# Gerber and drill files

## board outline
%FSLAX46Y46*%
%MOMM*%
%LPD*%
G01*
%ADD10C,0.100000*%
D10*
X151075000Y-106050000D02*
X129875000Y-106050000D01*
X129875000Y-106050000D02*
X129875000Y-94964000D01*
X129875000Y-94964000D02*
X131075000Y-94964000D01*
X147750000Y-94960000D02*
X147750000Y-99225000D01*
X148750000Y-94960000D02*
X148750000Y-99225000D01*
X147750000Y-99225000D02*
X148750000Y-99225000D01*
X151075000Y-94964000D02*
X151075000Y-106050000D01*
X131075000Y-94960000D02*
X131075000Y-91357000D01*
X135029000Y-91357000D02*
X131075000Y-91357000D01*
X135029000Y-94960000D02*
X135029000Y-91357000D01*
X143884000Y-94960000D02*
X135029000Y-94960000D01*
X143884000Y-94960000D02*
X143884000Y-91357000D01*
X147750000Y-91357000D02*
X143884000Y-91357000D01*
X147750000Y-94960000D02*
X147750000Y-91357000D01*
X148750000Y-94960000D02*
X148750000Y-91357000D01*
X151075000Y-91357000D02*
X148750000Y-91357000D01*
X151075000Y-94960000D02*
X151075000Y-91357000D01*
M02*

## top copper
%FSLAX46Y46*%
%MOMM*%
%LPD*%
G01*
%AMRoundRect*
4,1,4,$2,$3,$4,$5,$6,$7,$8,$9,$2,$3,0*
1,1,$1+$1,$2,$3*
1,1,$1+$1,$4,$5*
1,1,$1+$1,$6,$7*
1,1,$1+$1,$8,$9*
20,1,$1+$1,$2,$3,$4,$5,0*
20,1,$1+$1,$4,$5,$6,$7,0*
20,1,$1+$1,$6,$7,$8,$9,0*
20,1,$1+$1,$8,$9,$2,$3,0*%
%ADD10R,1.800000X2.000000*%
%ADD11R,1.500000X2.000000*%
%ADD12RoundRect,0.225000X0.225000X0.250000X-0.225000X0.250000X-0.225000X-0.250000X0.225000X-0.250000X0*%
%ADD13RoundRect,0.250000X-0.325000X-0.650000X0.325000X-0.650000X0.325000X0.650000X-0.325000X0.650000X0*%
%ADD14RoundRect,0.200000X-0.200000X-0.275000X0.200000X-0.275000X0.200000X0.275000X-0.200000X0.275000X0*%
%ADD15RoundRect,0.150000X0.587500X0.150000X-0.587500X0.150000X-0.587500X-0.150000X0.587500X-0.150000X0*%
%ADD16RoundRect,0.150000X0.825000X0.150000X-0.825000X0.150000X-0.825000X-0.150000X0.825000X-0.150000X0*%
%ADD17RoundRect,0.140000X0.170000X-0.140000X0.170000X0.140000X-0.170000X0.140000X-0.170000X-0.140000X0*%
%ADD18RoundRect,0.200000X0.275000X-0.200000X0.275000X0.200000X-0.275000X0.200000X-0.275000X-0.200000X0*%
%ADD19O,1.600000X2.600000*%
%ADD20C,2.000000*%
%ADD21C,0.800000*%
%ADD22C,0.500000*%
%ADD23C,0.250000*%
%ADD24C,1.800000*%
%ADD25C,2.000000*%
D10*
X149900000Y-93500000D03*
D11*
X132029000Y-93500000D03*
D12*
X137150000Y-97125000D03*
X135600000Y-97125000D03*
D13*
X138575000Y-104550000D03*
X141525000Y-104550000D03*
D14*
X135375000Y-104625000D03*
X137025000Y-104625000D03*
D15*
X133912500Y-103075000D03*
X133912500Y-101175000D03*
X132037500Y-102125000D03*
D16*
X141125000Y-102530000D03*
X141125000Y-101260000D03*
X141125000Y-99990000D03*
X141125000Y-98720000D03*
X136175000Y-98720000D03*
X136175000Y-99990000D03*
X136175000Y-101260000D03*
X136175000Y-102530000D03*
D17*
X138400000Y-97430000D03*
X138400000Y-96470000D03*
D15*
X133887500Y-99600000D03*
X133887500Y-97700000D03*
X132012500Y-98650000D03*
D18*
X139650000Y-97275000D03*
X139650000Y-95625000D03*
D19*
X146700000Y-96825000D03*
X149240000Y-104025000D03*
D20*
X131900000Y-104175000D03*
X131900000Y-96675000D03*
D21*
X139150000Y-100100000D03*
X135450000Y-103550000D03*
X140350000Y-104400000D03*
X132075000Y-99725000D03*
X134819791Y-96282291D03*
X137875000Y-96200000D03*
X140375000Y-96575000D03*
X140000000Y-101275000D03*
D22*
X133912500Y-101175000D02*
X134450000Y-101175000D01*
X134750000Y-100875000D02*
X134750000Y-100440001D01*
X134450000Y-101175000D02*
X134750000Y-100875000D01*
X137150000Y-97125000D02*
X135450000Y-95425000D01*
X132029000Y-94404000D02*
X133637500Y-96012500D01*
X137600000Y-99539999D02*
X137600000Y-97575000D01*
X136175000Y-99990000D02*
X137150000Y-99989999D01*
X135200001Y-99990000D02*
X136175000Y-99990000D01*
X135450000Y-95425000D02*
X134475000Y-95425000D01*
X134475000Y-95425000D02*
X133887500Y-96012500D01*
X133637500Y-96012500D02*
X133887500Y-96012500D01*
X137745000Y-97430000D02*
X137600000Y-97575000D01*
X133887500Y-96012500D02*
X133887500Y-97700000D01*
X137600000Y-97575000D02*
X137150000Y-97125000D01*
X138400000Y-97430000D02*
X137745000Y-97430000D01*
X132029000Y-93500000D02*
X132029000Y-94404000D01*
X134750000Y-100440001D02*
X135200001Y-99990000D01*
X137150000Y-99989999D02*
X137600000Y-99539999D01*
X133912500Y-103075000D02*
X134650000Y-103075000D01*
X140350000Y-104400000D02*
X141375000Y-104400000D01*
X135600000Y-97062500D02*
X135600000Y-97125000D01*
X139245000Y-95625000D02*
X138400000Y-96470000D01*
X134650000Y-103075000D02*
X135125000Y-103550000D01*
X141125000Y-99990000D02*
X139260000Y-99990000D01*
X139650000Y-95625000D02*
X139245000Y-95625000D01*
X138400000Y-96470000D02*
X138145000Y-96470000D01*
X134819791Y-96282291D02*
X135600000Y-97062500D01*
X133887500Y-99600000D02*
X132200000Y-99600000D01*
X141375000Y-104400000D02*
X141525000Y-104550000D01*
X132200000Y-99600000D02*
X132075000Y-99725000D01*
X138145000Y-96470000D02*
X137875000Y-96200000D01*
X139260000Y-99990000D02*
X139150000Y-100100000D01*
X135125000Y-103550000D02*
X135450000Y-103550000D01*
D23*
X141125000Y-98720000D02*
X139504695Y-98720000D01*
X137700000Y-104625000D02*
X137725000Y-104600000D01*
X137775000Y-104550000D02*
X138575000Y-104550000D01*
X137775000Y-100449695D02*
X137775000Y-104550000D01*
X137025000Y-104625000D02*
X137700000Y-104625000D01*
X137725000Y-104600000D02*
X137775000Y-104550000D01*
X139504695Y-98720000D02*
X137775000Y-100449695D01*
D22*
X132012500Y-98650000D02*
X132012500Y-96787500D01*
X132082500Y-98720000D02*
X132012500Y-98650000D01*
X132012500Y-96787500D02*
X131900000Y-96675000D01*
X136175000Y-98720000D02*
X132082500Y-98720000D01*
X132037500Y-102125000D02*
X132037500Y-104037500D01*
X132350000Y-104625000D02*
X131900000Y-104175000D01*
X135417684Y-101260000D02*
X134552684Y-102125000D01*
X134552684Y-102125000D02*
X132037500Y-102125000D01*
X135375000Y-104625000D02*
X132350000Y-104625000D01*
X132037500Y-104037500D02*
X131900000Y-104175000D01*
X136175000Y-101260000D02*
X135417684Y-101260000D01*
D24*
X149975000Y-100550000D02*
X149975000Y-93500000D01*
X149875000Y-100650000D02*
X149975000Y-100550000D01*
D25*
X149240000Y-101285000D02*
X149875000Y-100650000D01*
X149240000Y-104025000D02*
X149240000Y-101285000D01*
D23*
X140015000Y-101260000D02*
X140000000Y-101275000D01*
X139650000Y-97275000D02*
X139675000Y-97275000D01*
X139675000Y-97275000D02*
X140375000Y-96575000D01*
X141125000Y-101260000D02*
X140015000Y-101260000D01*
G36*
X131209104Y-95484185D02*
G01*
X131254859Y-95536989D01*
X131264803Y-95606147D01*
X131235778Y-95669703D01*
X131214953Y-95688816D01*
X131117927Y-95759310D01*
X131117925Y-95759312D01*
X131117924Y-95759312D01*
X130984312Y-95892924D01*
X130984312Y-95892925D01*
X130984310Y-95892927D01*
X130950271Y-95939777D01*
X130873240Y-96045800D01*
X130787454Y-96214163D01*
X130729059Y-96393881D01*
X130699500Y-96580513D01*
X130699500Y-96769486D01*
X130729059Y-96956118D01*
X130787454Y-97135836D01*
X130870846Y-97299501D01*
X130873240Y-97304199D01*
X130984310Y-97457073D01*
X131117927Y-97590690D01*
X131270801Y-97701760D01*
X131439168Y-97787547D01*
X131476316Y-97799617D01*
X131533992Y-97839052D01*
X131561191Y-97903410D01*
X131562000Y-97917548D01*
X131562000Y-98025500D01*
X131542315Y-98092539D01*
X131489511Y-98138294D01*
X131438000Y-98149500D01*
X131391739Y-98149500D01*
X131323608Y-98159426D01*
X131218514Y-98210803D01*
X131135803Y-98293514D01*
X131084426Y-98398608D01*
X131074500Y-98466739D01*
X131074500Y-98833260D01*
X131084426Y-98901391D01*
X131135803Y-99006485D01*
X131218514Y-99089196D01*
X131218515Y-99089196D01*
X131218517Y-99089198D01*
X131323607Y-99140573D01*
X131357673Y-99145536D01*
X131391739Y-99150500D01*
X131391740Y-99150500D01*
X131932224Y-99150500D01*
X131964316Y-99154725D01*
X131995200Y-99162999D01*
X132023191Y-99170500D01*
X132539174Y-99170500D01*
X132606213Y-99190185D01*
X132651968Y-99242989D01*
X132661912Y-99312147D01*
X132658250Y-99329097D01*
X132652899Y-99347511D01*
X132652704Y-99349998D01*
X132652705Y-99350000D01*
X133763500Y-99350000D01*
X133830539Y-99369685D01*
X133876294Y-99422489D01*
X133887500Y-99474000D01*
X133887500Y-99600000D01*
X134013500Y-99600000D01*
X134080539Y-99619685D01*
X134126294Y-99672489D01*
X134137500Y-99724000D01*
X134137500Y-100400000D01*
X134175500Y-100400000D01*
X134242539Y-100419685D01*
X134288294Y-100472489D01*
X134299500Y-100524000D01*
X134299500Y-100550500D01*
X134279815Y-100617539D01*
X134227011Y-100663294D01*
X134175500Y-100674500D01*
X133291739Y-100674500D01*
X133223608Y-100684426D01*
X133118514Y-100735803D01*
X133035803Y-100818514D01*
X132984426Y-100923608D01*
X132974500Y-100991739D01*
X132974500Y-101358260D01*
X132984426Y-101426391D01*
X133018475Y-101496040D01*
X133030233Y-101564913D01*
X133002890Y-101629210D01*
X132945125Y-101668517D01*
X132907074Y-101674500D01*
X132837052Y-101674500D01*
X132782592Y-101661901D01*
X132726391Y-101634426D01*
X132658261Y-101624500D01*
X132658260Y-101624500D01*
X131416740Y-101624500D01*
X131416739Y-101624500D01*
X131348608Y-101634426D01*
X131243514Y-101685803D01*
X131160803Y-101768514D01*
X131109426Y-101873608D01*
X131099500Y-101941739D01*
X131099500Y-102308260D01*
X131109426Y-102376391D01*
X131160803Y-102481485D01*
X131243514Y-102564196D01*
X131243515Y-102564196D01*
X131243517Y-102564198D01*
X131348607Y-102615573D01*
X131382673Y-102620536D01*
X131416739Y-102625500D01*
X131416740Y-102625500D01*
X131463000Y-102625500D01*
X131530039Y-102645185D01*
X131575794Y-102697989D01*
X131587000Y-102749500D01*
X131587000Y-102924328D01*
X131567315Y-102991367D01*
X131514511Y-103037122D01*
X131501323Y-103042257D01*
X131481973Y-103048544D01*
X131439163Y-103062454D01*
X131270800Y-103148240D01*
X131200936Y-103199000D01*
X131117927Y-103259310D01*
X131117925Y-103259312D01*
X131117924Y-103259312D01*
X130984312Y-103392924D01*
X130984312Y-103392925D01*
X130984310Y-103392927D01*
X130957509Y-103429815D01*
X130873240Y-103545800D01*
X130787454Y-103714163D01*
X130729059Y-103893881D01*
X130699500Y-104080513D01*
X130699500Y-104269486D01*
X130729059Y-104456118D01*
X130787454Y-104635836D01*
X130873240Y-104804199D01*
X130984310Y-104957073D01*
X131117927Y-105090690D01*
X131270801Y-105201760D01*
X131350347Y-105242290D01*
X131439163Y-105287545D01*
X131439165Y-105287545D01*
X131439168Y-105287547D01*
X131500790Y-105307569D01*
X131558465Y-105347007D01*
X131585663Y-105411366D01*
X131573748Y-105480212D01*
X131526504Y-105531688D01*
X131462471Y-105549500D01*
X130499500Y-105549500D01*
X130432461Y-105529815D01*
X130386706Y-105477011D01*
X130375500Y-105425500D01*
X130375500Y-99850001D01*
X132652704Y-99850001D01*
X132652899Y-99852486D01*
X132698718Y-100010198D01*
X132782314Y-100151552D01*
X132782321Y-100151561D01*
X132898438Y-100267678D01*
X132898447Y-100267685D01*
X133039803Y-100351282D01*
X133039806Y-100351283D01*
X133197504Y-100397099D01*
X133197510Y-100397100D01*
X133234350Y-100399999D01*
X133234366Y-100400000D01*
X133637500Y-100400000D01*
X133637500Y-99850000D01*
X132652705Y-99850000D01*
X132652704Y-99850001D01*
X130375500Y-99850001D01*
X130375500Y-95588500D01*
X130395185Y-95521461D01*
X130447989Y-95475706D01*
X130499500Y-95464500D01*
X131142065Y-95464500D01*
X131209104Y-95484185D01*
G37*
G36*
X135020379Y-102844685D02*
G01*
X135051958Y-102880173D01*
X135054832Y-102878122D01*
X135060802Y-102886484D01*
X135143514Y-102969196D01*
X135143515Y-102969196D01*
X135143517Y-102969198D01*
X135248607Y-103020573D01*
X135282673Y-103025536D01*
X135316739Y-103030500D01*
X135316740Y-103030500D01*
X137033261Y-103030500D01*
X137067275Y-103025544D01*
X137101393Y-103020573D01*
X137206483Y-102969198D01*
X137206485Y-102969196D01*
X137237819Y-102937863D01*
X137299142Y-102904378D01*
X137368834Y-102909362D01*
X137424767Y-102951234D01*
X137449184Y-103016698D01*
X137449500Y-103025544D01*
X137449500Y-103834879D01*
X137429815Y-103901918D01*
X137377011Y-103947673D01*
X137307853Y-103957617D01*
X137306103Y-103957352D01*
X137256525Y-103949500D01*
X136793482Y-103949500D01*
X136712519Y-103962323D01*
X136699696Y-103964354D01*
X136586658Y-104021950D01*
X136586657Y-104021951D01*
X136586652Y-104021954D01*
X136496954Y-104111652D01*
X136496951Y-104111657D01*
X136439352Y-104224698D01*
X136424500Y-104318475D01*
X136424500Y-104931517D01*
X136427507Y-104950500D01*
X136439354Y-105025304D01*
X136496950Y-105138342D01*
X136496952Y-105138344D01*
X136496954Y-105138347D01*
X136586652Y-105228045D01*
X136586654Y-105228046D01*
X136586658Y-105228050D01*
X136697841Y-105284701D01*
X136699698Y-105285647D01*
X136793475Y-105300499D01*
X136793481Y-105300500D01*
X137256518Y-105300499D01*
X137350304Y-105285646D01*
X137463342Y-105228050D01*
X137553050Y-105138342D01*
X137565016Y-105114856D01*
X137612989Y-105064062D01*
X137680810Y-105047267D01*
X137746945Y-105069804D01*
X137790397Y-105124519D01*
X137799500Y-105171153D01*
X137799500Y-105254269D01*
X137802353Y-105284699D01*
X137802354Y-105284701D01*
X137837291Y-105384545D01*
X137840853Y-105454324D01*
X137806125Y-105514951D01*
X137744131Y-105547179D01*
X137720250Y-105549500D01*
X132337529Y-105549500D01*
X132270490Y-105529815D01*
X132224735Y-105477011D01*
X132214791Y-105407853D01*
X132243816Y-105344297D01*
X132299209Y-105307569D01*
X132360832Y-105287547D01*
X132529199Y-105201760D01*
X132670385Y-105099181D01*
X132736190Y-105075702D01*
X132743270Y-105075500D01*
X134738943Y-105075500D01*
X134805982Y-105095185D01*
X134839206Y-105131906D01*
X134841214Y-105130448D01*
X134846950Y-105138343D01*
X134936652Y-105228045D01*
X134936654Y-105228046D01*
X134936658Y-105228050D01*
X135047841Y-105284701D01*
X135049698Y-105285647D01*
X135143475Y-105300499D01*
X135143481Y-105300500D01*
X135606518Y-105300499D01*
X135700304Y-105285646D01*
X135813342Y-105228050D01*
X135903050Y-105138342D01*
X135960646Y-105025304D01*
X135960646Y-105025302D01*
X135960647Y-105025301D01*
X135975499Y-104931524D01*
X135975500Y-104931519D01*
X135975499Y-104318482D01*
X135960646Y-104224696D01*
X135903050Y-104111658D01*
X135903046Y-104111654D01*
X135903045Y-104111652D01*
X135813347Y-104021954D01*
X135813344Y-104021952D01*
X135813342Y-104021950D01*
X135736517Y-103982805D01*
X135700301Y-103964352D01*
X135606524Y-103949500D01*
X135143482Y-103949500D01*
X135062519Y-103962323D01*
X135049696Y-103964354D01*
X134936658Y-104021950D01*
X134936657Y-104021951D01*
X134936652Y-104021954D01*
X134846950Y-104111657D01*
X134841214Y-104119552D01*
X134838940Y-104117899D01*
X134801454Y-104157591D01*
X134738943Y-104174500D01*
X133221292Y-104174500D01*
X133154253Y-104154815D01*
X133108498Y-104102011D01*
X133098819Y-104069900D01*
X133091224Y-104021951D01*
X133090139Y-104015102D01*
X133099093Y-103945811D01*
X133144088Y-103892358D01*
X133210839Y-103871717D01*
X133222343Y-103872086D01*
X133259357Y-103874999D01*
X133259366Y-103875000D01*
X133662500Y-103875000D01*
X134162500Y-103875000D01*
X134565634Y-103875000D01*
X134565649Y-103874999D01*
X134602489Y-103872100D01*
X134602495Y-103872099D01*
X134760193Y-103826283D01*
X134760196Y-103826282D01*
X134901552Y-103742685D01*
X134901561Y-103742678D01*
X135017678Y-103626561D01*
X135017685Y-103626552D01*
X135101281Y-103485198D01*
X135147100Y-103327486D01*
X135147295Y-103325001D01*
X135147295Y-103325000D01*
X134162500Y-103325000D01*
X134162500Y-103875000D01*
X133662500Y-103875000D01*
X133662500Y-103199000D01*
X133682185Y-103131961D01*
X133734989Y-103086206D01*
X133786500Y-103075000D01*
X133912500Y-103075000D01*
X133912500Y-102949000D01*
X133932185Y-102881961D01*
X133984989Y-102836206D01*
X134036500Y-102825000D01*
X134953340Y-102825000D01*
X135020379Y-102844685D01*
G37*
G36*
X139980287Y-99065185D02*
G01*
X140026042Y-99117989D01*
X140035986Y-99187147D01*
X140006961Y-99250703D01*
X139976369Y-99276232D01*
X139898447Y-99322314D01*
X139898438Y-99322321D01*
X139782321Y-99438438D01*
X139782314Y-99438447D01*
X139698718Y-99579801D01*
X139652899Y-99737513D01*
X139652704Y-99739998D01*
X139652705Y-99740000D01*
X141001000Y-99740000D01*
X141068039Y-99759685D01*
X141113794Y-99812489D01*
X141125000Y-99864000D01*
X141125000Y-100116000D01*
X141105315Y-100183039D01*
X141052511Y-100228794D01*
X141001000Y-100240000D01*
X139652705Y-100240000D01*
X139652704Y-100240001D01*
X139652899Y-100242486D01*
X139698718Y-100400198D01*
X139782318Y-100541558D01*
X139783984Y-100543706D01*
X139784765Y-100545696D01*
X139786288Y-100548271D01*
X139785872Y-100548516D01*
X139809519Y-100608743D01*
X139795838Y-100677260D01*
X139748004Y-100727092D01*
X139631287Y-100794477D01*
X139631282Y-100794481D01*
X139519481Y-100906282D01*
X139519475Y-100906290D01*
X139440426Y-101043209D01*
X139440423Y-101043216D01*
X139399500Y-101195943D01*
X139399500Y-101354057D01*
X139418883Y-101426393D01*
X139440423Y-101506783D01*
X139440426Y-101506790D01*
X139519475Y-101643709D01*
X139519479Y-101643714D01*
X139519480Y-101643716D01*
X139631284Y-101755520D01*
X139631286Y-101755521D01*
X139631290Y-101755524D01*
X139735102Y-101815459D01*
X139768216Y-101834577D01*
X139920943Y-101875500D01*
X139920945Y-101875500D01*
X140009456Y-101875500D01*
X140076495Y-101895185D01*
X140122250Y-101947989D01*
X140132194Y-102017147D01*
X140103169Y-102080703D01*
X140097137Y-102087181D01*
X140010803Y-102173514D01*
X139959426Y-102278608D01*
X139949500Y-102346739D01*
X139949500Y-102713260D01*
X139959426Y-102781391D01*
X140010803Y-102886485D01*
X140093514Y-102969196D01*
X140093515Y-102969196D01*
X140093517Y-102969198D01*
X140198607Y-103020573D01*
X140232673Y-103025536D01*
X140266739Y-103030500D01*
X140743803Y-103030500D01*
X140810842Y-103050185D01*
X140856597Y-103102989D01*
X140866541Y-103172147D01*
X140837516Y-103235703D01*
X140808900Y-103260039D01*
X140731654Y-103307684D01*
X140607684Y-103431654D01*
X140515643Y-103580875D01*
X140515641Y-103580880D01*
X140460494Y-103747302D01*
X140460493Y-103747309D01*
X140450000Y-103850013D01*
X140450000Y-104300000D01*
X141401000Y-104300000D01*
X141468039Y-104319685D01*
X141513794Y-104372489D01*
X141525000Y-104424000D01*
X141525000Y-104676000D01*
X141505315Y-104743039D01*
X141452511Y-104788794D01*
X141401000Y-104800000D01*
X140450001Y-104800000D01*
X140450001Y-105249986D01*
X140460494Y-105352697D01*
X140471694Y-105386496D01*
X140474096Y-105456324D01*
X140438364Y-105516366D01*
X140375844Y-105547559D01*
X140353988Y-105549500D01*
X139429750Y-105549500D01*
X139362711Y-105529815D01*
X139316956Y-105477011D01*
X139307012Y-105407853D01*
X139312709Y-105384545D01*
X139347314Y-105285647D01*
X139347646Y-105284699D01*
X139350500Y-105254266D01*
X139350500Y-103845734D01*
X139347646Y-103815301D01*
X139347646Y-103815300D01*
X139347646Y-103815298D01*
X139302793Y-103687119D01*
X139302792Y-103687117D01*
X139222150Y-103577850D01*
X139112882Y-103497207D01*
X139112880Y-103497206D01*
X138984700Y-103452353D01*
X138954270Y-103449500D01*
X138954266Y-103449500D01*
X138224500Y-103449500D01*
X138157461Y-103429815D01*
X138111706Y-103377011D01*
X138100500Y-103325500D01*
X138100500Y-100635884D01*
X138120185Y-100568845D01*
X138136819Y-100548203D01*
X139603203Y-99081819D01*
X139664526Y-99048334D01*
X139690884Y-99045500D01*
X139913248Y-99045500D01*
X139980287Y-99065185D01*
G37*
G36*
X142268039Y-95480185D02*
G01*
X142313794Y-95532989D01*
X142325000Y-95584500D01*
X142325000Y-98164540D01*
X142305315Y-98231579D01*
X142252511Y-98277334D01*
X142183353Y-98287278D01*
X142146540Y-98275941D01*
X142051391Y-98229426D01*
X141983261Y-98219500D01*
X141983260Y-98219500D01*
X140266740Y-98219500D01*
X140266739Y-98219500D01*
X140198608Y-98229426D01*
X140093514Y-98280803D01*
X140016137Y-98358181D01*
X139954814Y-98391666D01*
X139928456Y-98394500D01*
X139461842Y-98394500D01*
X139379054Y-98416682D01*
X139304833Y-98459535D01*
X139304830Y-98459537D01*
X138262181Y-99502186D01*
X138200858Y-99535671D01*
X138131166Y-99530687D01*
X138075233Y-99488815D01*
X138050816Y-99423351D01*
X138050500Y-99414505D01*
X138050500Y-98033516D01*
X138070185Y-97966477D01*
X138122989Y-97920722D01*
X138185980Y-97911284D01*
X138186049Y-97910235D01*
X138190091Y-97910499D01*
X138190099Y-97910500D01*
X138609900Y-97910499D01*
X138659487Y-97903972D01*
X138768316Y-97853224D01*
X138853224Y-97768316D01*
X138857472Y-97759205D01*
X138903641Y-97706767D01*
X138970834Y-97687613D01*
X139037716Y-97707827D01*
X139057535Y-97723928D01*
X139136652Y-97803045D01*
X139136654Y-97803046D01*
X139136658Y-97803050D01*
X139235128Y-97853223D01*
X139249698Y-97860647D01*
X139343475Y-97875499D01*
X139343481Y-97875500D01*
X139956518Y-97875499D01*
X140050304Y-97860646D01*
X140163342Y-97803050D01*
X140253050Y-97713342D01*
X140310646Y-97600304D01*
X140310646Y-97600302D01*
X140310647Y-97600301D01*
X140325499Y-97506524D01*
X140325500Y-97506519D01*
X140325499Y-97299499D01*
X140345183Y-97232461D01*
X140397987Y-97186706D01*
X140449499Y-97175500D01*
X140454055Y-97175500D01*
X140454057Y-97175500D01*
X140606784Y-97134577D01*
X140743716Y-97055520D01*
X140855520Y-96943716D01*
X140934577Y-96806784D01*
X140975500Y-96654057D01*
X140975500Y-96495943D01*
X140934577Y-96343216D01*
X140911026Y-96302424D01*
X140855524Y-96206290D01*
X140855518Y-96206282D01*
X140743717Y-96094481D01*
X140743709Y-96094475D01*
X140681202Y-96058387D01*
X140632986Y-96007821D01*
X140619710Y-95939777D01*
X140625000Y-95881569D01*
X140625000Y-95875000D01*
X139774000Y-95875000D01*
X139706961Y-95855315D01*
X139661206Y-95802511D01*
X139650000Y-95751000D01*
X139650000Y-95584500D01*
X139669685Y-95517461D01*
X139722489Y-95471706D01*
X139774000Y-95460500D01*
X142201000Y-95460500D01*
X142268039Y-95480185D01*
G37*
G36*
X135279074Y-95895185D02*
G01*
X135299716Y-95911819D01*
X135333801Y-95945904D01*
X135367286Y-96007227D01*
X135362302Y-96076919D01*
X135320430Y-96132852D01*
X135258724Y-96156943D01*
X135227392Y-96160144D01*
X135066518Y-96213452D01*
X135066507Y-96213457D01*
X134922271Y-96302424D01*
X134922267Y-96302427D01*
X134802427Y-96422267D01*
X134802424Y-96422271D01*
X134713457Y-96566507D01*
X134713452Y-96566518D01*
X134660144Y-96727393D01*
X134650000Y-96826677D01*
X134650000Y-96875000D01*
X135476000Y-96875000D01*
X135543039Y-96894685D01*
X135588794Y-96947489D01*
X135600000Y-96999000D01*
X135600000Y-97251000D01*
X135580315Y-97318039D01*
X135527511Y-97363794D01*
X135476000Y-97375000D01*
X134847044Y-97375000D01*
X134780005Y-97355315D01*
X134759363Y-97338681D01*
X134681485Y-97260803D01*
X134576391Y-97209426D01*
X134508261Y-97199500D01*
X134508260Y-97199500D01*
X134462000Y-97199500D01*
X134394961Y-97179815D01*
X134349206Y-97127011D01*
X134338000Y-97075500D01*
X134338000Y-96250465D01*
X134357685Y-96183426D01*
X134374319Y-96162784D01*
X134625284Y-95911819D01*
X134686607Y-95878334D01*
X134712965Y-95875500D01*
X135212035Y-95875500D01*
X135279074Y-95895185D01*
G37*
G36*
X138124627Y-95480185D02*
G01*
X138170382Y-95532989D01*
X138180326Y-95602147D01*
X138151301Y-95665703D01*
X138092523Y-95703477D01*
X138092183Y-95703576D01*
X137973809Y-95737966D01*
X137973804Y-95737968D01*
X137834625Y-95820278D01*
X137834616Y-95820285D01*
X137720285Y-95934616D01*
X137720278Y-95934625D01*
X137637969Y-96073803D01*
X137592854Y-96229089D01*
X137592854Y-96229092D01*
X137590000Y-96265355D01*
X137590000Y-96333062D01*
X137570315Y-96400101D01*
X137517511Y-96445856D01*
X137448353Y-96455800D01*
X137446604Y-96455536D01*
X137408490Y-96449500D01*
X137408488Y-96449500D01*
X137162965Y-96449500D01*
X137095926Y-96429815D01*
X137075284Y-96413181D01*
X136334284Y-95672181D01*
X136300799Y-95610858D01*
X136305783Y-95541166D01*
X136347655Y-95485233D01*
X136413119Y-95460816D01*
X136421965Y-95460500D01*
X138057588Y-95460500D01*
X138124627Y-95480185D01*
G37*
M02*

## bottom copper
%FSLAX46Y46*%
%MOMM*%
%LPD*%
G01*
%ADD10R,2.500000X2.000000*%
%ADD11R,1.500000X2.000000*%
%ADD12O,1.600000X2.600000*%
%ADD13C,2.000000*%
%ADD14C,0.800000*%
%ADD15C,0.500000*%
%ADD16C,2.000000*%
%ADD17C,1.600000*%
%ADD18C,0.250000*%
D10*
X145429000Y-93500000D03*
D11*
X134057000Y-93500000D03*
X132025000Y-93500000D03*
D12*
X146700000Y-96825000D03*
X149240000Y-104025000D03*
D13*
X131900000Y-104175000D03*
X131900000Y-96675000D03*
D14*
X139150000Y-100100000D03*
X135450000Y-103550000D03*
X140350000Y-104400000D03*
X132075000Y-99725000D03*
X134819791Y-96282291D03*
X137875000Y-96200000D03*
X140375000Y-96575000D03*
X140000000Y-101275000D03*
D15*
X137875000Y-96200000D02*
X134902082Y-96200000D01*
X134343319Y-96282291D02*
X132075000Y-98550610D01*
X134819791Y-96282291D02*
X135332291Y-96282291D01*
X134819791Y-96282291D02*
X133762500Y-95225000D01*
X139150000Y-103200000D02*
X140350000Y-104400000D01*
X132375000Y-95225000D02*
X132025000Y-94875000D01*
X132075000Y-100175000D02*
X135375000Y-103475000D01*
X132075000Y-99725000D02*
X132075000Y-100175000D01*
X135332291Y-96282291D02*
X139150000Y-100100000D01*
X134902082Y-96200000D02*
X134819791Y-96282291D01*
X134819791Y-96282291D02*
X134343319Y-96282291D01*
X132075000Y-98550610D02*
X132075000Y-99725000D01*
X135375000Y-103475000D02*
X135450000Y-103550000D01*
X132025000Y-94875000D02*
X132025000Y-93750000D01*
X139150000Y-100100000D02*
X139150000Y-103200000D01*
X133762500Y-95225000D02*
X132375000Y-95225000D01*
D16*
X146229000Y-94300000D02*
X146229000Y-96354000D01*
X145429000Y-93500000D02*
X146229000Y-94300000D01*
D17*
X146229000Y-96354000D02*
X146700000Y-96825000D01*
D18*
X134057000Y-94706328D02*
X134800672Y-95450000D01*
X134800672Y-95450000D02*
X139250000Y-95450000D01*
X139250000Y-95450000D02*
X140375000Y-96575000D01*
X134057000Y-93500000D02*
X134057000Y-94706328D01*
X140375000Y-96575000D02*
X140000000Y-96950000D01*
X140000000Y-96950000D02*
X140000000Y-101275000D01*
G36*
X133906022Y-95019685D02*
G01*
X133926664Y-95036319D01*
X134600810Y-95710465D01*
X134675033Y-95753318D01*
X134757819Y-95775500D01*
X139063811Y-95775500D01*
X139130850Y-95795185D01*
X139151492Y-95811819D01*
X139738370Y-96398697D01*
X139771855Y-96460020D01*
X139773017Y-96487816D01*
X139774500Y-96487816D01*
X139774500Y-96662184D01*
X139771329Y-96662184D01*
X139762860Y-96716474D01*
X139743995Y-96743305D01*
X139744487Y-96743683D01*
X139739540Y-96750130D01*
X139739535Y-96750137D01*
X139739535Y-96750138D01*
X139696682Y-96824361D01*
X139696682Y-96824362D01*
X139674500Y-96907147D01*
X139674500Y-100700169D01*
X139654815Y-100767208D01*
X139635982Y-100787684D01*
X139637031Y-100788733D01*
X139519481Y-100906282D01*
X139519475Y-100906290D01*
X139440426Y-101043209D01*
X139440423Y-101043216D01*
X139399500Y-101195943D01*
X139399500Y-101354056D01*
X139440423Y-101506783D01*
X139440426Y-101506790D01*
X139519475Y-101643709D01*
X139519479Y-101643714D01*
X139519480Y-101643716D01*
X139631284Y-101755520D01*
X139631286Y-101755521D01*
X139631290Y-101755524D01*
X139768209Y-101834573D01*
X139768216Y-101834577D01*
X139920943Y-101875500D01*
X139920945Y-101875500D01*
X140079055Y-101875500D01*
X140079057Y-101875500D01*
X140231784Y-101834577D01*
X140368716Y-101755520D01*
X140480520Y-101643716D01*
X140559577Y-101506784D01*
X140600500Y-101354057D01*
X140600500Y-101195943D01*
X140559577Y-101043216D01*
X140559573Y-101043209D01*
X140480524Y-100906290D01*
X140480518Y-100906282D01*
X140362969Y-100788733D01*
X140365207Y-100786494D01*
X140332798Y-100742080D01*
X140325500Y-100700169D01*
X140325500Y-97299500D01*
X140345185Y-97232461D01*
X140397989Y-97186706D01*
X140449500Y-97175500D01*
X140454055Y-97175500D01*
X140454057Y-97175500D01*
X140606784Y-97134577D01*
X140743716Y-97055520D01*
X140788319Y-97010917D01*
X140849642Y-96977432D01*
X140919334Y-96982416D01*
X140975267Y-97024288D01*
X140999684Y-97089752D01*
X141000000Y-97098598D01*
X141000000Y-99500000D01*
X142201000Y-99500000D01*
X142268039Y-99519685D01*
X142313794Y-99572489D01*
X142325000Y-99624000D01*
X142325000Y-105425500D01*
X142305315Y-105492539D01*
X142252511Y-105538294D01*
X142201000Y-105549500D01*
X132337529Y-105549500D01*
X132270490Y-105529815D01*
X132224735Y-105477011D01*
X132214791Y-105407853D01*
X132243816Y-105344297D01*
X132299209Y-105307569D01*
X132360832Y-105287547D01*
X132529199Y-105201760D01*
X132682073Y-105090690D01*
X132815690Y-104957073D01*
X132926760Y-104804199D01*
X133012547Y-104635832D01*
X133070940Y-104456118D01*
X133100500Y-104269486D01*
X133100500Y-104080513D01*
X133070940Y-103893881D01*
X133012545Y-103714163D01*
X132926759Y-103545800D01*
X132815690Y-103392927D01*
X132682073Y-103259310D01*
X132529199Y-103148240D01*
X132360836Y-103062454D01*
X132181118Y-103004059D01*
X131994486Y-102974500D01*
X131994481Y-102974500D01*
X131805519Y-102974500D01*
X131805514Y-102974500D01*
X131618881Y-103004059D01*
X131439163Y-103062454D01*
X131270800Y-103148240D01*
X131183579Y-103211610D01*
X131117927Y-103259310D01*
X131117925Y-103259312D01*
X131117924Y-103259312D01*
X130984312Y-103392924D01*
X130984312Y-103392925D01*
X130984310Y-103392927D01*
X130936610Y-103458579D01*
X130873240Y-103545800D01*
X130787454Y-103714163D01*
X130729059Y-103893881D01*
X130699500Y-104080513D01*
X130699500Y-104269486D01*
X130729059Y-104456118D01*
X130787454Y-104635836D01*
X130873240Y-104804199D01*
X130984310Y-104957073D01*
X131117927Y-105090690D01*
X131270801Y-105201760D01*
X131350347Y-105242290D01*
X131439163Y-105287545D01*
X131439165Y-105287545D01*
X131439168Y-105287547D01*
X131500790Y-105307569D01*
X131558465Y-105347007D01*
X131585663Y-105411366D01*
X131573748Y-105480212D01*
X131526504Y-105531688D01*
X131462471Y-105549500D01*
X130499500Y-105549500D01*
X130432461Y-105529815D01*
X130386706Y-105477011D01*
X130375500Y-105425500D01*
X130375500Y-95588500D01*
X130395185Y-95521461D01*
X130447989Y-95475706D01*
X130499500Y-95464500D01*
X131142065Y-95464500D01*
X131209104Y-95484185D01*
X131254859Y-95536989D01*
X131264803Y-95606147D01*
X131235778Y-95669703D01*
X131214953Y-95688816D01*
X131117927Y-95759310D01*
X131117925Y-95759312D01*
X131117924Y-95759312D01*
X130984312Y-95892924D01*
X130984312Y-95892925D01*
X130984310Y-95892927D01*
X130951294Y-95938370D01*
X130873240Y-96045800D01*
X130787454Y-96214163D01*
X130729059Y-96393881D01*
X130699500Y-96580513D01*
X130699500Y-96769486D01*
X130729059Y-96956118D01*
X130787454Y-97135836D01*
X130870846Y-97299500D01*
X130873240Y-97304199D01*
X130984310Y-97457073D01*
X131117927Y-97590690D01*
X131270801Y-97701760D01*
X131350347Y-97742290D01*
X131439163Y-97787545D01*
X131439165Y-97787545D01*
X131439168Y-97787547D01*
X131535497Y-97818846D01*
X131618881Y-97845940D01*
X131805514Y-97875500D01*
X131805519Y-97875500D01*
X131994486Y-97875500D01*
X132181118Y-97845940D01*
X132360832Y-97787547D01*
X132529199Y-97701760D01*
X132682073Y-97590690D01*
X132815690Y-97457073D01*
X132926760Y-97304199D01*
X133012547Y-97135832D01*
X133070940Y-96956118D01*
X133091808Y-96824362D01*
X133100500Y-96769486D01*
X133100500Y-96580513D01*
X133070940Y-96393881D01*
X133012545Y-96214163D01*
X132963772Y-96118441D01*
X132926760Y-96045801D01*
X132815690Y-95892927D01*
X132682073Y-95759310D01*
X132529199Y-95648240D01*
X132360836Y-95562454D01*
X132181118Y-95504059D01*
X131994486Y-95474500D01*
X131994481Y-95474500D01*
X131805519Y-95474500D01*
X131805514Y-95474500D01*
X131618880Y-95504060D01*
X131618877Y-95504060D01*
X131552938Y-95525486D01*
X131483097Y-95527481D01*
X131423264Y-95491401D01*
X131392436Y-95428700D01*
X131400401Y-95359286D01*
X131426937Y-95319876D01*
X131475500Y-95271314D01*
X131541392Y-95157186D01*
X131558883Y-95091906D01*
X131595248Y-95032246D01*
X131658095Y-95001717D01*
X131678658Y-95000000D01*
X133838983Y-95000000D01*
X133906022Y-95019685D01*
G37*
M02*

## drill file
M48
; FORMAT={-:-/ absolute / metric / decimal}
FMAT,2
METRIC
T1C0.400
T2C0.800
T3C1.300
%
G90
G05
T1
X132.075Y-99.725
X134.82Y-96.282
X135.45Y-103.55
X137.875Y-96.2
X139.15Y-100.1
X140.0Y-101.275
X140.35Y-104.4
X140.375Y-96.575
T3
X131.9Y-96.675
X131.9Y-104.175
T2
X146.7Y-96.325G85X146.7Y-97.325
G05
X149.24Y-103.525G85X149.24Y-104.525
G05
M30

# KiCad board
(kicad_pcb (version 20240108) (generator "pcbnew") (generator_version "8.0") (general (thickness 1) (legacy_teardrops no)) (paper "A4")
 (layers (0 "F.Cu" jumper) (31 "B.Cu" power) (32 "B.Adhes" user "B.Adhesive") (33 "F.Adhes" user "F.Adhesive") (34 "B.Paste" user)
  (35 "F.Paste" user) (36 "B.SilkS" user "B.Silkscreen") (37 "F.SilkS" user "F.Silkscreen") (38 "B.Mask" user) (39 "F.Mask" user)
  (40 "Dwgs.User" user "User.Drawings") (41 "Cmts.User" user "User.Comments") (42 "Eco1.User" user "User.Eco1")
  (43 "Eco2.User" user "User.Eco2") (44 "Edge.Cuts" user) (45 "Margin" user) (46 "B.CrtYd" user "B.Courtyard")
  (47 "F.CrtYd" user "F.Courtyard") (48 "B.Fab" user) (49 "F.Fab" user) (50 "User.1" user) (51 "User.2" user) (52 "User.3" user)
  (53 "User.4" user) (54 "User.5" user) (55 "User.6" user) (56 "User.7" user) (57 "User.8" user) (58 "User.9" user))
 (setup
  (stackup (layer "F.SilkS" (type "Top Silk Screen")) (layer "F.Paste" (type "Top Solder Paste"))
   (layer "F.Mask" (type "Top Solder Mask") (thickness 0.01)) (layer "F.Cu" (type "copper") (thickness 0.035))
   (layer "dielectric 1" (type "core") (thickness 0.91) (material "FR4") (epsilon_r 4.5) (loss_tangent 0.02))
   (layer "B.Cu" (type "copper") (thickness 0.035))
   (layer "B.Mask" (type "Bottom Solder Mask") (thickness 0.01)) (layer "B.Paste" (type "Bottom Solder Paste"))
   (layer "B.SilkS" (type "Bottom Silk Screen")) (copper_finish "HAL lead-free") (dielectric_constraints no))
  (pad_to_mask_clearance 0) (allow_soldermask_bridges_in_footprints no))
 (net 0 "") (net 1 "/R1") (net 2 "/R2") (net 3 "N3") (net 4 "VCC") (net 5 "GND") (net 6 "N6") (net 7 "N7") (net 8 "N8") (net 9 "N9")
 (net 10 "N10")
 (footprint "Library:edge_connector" (layer "F.Cu") (at 151.329 92.23 180)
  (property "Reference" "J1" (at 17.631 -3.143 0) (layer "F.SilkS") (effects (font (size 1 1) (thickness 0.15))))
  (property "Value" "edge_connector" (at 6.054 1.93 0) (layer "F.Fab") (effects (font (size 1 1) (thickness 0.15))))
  (fp_line (start 20.254 -2.73) (end 20.254 0.873) (stroke (width 0.1) (type solid)) (layer "Edge.Cuts"))
  (fp_line (start 16.3 0.873) (end 20.254 0.873) (stroke (width 0.1) (type solid)) (layer "Edge.Cuts"))
  (fp_line (start 16.3 -2.73) (end 16.3 0.873) (stroke (width 0.1) (type solid)) (layer "Edge.Cuts"))
  (fp_line (start 7.445 -2.73) (end 16.3 -2.73) (stroke (width 0.1) (type solid)) (layer "Edge.Cuts"))
  (fp_line (start 7.445 -2.73) (end 7.445 0.873) (stroke (width 0.1) (type solid)) (layer "Edge.Cuts"))
  (fp_line (start 3.579 0.873) (end 7.445 0.873) (stroke (width 0.1) (type solid)) (layer "Edge.Cuts"))
  (fp_line (start 3.579 -2.73) (end 3.579 0.873) (stroke (width 0.1) (type solid)) (layer "Edge.Cuts"))
  (fp_line (start 2.579 -2.73) (end 2.579 0.873) (stroke (width 0.1) (type solid)) (layer "Edge.Cuts"))
  (fp_line (start 0.254 0.873) (end 2.579 0.873) (stroke (width 0.1) (type solid)) (layer "Edge.Cuts"))
  (fp_line (start 0.254 -2.73) (end 0.254 0.873) (stroke (width 0.1) (type solid)) (layer "Edge.Cuts"))
  (pad "1" connect rect (at 1.429 -1.27 180) (size 1.8 2) (layers "F.Cu" "F.Mask") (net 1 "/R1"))
  (pad "2" connect rect (at 5.9 -1.27 180) (size 2.5 2) (layers "B.Cu" "B.Mask") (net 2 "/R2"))
  (pad "3" connect rect (at 17.272 -1.27 180) (size 1.5 2) (layers "B.Cu" "B.Mask") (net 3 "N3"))
  (pad "4" connect rect (at 19.3 -1.27 180) (size 1.5 2) (layers "F.Cu" "F.Mask") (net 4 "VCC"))
  (pad "5" connect rect (at 19.304 -1.27 180) (size 1.5 2) (layers "B.Cu" "B.Mask") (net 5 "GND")))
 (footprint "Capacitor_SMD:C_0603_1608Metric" (layer "F.Cu") (at 136.375 97.125 180)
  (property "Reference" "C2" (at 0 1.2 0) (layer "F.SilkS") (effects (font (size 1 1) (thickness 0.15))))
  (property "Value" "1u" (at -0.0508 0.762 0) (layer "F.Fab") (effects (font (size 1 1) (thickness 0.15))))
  (pad "1" smd roundrect (at -0.775 0 180) (size 0.9 0.95) (layers "F.Cu" "F.Paste" "F.Mask") (roundrect_rratio 0.25) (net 4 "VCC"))
  (pad "2" smd roundrect (at 0.775 0 180) (size 0.9 0.95) (layers "F.Cu" "F.Paste" "F.Mask") (roundrect_rratio 0.25) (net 5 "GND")))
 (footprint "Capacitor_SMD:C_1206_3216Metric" (layer "F.Cu") (at 140.05 104.55)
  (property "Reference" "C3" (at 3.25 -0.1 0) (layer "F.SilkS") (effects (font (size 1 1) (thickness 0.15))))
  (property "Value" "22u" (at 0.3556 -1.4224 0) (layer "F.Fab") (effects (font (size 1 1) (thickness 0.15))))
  (pad "1" smd roundrect (at -1.475 0) (size 1.15 1.8) (layers "F.Cu" "F.Paste" "F.Mask") (roundrect_rratio 0.2173913043) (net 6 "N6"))
  (pad "2" smd roundrect (at 1.475 0) (size 1.15 1.8) (layers "F.Cu" "F.Paste" "F.Mask") (roundrect_rratio 0.2173913043) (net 5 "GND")))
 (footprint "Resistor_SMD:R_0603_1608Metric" (layer "F.Cu") (at 136.2 104.625)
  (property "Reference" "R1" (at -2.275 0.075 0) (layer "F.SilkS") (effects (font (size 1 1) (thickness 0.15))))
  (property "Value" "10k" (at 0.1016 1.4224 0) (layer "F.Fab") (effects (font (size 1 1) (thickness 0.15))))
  (pad "1" smd roundrect (at -0.825 0) (size 0.8 0.95) (layers "F.Cu" "F.Paste" "F.Mask") (roundrect_rratio 0.25) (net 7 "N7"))
  (pad "2" smd roundrect (at 0.825 0) (size 0.8 0.95) (layers "F.Cu" "F.Paste" "F.Mask") (roundrect_rratio 0.25) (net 6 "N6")))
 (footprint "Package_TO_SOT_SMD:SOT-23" (layer "F.Cu") (at 132.975 102.125 180)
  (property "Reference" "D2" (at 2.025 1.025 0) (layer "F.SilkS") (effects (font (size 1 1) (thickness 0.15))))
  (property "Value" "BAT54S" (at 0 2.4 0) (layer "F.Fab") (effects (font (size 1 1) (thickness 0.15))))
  (pad "1" smd roundrect (at -0.9375 -0.95 180) (size 1.475 0.6) (layers "F.Cu" "F.Paste" "F.Mask") (roundrect_rratio 0.25) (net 5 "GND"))
  (pad "2" smd roundrect (at -0.9375 0.95 180) (size 1.475 0.6) (layers "F.Cu" "F.Paste" "F.Mask") (roundrect_rratio 0.25) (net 4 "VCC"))
  (pad "3" smd roundrect (at 0.9375 0 180) (size 1.475 0.6) (layers "F.Cu" "F.Paste" "F.Mask") (roundrect_rratio 0.25) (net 7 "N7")))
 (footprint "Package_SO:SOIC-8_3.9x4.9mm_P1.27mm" (layer "F.Cu") (at 138.65 100.625 180)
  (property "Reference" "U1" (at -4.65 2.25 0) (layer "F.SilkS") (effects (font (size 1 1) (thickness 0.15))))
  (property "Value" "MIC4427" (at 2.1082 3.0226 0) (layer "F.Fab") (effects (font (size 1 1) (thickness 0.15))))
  (pad "1" smd roundrect (at -2.475 -1.905 180) (size 1.95 0.6) (layers "F.Cu" "F.Paste" "F.Mask") (roundrect_rratio 0.25) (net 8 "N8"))
  (pad "2" smd roundrect (at -2.475 -0.635 180) (size 1.95 0.6) (layers "F.Cu" "F.Paste" "F.Mask") (roundrect_rratio 0.25) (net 3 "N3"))
  (pad "3" smd roundrect (at -2.475 0.635 180) (size 1.95 0.6) (layers "F.Cu" "F.Paste" "F.Mask") (roundrect_rratio 0.25) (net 5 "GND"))
  (pad "4" smd roundrect (at -2.475 1.905 180) (size 1.95 0.6) (layers "F.Cu" "F.Paste" "F.Mask") (roundrect_rratio 0.25) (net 6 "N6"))
  (pad "5" smd roundrect (at 2.475 1.905 180) (size 1.95 0.6) (layers "F.Cu" "F.Paste" "F.Mask") (roundrect_rratio 0.25) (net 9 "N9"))
  (pad "6" smd roundrect (at 2.475 0.635 180) (size 1.95 0.6) (layers "F.Cu" "F.Paste" "F.Mask") (roundrect_rratio 0.25) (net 4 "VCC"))
  (pad "7" smd roundrect (at 2.475 -0.635 180) (size 1.95 0.6) (layers "F.Cu" "F.Paste" "F.Mask") (roundrect_rratio 0.25) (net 7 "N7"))
  (pad "8" smd roundrect (at 2.475 -1.905 180) (size 1.95 0.6) (layers "F.Cu" "F.Paste" "F.Mask") (roundrect_rratio 0.25) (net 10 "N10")))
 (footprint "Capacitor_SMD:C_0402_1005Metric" (layer "F.Cu") (at 138.4 96.95 90)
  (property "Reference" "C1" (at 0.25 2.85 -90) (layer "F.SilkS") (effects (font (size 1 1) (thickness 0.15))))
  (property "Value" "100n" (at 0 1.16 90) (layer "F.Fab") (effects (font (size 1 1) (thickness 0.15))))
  (pad "1" smd roundrect (at -0.48 0 90) (size 0.56 0.62) (layers "F.Cu" "F.Paste" "F.Mask") (roundrect_rratio 0.25) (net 4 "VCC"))
  (pad "2" smd roundrect (at 0.48 0 90) (size 0.56 0.62) (layers "F.Cu" "F.Paste" "F.Mask") (roundrect_rratio 0.25) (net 5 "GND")))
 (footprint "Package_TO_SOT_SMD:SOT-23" (layer "F.Cu") (at 132.95 98.65 180)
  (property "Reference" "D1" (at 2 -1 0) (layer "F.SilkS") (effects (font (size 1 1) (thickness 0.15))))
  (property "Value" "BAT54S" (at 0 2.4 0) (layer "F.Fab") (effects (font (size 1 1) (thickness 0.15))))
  (pad "1" smd roundrect (at -0.9375 -0.95 180) (size 1.475 0.6) (layers "F.Cu" "F.Paste" "F.Mask") (roundrect_rratio 0.25) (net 5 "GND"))
  (pad "2" smd roundrect (at -0.9375 0.95 180) (size 1.475 0.6) (layers "F.Cu" "F.Paste" "F.Mask") (roundrect_rratio 0.25) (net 4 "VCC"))
  (pad "3" smd roundrect (at 0.9375 0 180) (size 1.475 0.6) (layers "F.Cu" "F.Paste" "F.Mask") (roundrect_rratio 0.25) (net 9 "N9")))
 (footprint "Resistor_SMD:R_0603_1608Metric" (layer "F.Cu") (at 139.65 96.45 90)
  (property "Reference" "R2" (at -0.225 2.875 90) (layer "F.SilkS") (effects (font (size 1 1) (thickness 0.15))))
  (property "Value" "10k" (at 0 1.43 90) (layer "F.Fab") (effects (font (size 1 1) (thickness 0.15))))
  (pad "1" smd roundrect (at -0.825 0 90) (size 0.8 0.95) (layers "F.Cu" "F.Paste" "F.Mask") (roundrect_rratio 0.25) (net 3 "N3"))
  (pad "2" smd roundrect (at 0.825 0 90) (size 0.8 0.95) (layers "F.Cu" "F.Paste" "F.Mask") (roundrect_rratio 0.25) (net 5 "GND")))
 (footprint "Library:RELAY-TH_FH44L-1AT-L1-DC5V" (layer "B.Cu") (at 140.57 100.425)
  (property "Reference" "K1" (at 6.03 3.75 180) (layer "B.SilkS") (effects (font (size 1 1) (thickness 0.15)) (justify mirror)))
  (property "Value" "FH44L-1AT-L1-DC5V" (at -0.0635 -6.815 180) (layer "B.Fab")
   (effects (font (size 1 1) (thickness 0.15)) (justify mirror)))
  (pad "13" thru_hole oval (at 6.13 -3.6) (size 1.6 2.6) (drill oval 0.8 1.8) (layers "*.Cu" "*.Mask") (remove_unused_layers no)
   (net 2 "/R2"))
  (pad "14" thru_hole oval (at 8.67 3.6) (size 1.6 2.6) (drill oval 0.8 1.8) (layers "*.Cu" "*.Mask") (remove_unused_layers no)
   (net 1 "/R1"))
  (pad "A1" thru_hole circle (at -8.67 3.75) (size 2 2) (drill 1.3) (layers "*.Cu" "*.Mask") (remove_unused_layers no) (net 7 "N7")
   (thermal_bridge_angle 90))
  (pad "A2" thru_hole circle (at -8.67 -3.75) (size 2 2) (drill 1.3) (layers "*.Cu" "*.Mask") (remove_unused_layers no) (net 9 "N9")
   (thermal_bridge_angle 90)))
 (gr_line (start 151.075 106.05) (end 129.875 106.05) (stroke (width 0.1) (type solid)) (layer "Edge.Cuts"))
 (gr_line (start 129.875 106.05) (end 129.875 94.964) (stroke (width 0.1) (type solid)) (layer "Edge.Cuts"))
 (gr_line (start 129.875 94.964) (end 131.075 94.964) (stroke (width 0.1) (type solid)) (layer "Edge.Cuts"))
 (gr_line (start 147.75 94.96) (end 147.75 99.225) (stroke (width 0.1) (type default)) (layer "Edge.Cuts"))
 (gr_line (start 148.75 94.96) (end 148.75 99.225) (stroke (width 0.1) (type default)) (layer "Edge.Cuts"))
 (gr_line (start 147.75 99.225) (end 148.75 99.225) (stroke (width 0.1) (type default)) (layer "Edge.Cuts"))
 (gr_line (start 151.075 94.964) (end 151.075 106.05) (stroke (width 0.1) (type solid)) (layer "Edge.Cuts"))
 (segment (start 133.9125 101.175) (end 134.45 101.175) (width 0.5) (layer "F.Cu") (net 4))
 (segment (start 134.75 100.875) (end 134.75 100.440001) (width 0.5) (layer "F.Cu") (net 4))
 (segment (start 134.45 101.175) (end 134.75 100.875) (width 0.5) (layer "F.Cu") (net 4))
 (segment (start 137.15 97.125) (end 135.45 95.425) (width 0.5) (layer "F.Cu") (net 4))
 (segment (start 132.029 94.404) (end 133.6375 96.0125) (width 0.5) (layer "F.Cu") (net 4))
 (segment (start 137.6 99.539999) (end 137.6 97.575) (width 0.5) (layer "F.Cu") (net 4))
 (segment (start 136.175 99.99) (end 137.15 99.989999) (width 0.5) (layer "F.Cu") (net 4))
 (segment (start 135.200001 99.99) (end 136.175 99.99) (width 0.5) (layer "F.Cu") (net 4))
 (segment (start 135.45 95.425) (end 134.475 95.425) (width 0.5) (layer "F.Cu") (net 4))
 (segment (start 134.475 95.425) (end 133.8875 96.0125) (width 0.5) (layer "F.Cu") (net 4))
 (segment (start 133.6375 96.0125) (end 133.8875 96.0125) (width 0.5) (layer "F.Cu") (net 4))
 (segment (start 137.745 97.43) (end 137.6 97.575) (width 0.5) (layer "F.Cu") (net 4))
 (segment (start 133.8875 96.0125) (end 133.8875 97.7) (width 0.5) (layer "F.Cu") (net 4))
 (segment (start 137.6 97.575) (end 137.15 97.125) (width 0.5) (layer "F.Cu") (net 4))
 (segment (start 138.4 97.43) (end 137.745 97.43) (width 0.5) (layer "F.Cu") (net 4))
 (segment (start 132.029 93.5) (end 132.029 94.404) (width 0.5) (layer "F.Cu") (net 4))
 (segment (start 134.75 100.440001) (end 135.200001 99.99) (width 0.5) (layer "F.Cu") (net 4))
 (segment (start 137.15 99.989999) (end 137.6 99.539999) (width 0.5) (layer "F.Cu") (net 4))
 (segment (start 133.9125 103.075) (end 134.65 103.075) (width 0.5) (layer "F.Cu") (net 5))
 (segment (start 140.35 104.4) (end 141.375 104.4) (width 0.5) (layer "F.Cu") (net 5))
 (segment (start 135.6 97.0625) (end 135.6 97.125) (width 0.5) (layer "F.Cu") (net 5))
 (segment (start 139.245 95.625) (end 138.4 96.47) (width 0.5) (layer "F.Cu") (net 5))
 (segment (start 134.65 103.075) (end 135.125 103.55) (width 0.5) (layer "F.Cu") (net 5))
 (segment (start 141.125 99.99) (end 139.26 99.99) (width 0.5) (layer "F.Cu") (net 5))
 (segment (start 139.65 95.625) (end 139.245 95.625) (width 0.5) (layer "F.Cu") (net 5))
 (segment (start 138.4 96.47) (end 138.145 96.47) (width 0.5) (layer "F.Cu") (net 5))
 (segment (start 134.819791 96.282291) (end 135.6 97.0625) (width 0.5) (layer "F.Cu") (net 5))
 (segment (start 133.8875 99.6) (end 132.2 99.6) (width 0.5) (layer "F.Cu") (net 5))
 (segment (start 141.375 104.4) (end 141.525 104.55) (width 0.5) (layer "F.Cu") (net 5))
 (segment (start 132.2 99.6) (end 132.075 99.725) (width 0.5) (layer "F.Cu") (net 5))
 (segment (start 138.145 96.47) (end 137.875 96.2) (width 0.5) (layer "F.Cu") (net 5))
 (segment (start 139.26 99.99) (end 139.15 100.1) (width 0.5) (layer "F.Cu") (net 5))
 (segment (start 135.125 103.55) (end 135.45 103.55) (width 0.5) (layer "F.Cu") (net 5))
 (via (at 139.15 100.1) (size 0.8) (drill 0.4) (layers "F.Cu" "B.Cu") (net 5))
 (via (at 135.45 103.55) (size 0.8) (drill 0.4) (layers "F.Cu" "B.Cu") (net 5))
 (via (at 140.35 104.4) (size 0.8) (drill 0.4) (layers "F.Cu" "B.Cu") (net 5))
 (via (at 132.075 99.725) (size 0.8) (drill 0.4) (layers "F.Cu" "B.Cu") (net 5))
 (via (at 134.819791 96.282291) (size 0.8) (drill 0.4) (layers "F.Cu" "B.Cu") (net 5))
 (via (at 137.875 96.2) (size 0.8) (drill 0.4) (layers "F.Cu" "B.Cu") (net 5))
 (segment (start 137.875 96.2) (end 134.902082 96.2) (width 0.5) (layer "B.Cu") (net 5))
 (segment (start 134.343319 96.282291) (end 132.075 98.55061) (width 0.5) (layer "B.Cu") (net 5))
 (segment (start 134.819791 96.282291) (end 135.332291 96.282291) (width 0.5) (layer "B.Cu") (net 5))
 (segment (start 134.819791 96.282291) (end 133.7625 95.225) (width 0.5) (layer "B.Cu") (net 5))
 (segment (start 139.15 103.2) (end 140.35 104.4) (width 0.5) (layer "B.Cu") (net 5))
 (segment (start 132.375 95.225) (end 132.025 94.875) (width 0.5) (layer "B.Cu") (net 5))
 (segment (start 132.075 100.175) (end 135.375 103.475) (width 0.5) (layer "B.Cu") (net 5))
 (segment (start 132.075 99.725) (end 132.075 100.175) (width 0.5) (layer "B.Cu") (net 5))
 (segment (start 135.332291 96.282291) (end 139.15 100.1) (width 0.5) (layer "B.Cu") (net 5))
 (segment (start 134.902082 96.2) (end 134.819791 96.282291) (width 0.5) (layer "B.Cu") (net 5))
 (segment (start 134.819791 96.282291) (end 134.343319 96.282291) (width 0.5) (layer "B.Cu") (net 5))
 (segment (start 132.075 98.55061) (end 132.075 99.725) (width 0.5) (layer "B.Cu") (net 5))
 (segment (start 135.375 103.475) (end 135.45 103.55) (width 0.5) (layer "B.Cu") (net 5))
 (segment (start 132.025 94.875) (end 132.025 93.75) (width 0.5) (layer "B.Cu") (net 5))
 (segment (start 139.15 100.1) (end 139.15 103.2) (width 0.5) (layer "B.Cu") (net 5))
 (segment (start 133.7625 95.225) (end 132.375 95.225) (width 0.5) (layer "B.Cu") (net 5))
 (segment (start 141.125 98.72) (end 139.504695 98.72) (width 0.25) (layer "F.Cu") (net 6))
 (segment (start 137.7 104.625) (end 137.725 104.6) (width 0.25) (layer "F.Cu") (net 6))
 (segment (start 137.775 104.55) (end 138.575 104.55) (width 0.25) (layer "F.Cu") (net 6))
 (segment (start 137.775 100.449695) (end 137.775 104.55) (width 0.25) (layer "F.Cu") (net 6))
 (segment (start 137.025 104.625) (end 137.7 104.625) (width 0.25) (layer "F.Cu") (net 6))
 (segment (start 137.725 104.6) (end 137.775 104.55) (width 0.25) (layer "F.Cu") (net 6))
 (segment (start 139.504695 98.72) (end 137.775 100.449695) (width 0.25) (layer "F.Cu") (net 6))
 (segment (start 132.0125 98.65) (end 132.0125 96.7875) (width 0.5) (layer "F.Cu") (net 9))
 (segment (start 132.0825 98.72) (end 132.0125 98.65) (width 0.5) (layer "F.Cu") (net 9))
 (segment (start 132.0125 96.7875) (end 131.9 96.675) (width 0.5) (layer "F.Cu") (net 9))
 (segment (start 136.175 98.72) (end 132.0825 98.72) (width 0.5) (layer "F.Cu") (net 9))
 (segment (start 132.0375 102.125) (end 132.0375 104.0375) (width 0.5) (layer "F.Cu") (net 7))
 (segment (start 132.35 104.625) (end 131.9 104.175) (width 0.5) (layer "F.Cu") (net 7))
 (segment (start 135.417684 101.26) (end 134.552684 102.125) (width 0.5) (layer "F.Cu") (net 7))
 (segment (start 134.552684 102.125) (end 132.0375 102.125) (width 0.5) (layer "F.Cu") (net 7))
 (segment (start 135.375 104.625) (end 132.35 104.625) (width 0.5) (layer "F.Cu") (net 7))
 (segment (start 132.0375 104.0375) (end 131.9 104.175) (width 0.5) (layer "F.Cu") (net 7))
 (segment (start 136.175 101.26) (end 135.417684 101.26) (width 0.5) (layer "F.Cu") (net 7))
 (segment (start 146.229 94.3) (end 146.229 96.354) (width 2) (layer "B.Cu") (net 2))
 (segment (start 145.429 93.5) (end 146.229 94.3) (width 2) (layer "B.Cu") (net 2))
 (segment (start 146.229 96.354) (end 146.7 96.825) (width 1.6) (layer "B.Cu") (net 2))
 (segment (start 149.975 100.55) (end 149.975 93.5) (width 1.8) (layer "F.Cu") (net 1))
 (segment (start 149.875 100.65) (end 149.975 100.55) (width 1.8) (layer "F.Cu") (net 1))
 (segment (start 149.24 101.285) (end 149.875 100.65) (width 2) (layer "F.Cu") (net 1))
 (segment (start 149.24 104.025) (end 149.24 101.285) (width 2) (layer "F.Cu") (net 1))
 (segment (start 140.015 101.26) (end 140 101.275) (width 0.25) (layer "F.Cu") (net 3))
 (segment (start 139.65 97.275) (end 139.675 97.275) (width 0.25) (layer "F.Cu") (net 3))
 (segment (start 139.675 97.275) (end 140.375 96.575) (width 0.25) (layer "F.Cu") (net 3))
 (segment (start 141.125 101.26) (end 140.015 101.26) (width 0.25) (layer "F.Cu") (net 3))
 (via (at 140.375 96.575) (size 0.8) (drill 0.4) (layers "F.Cu" "B.Cu") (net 3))
 (via (at 140 101.275) (size 0.8) (drill 0.4) (layers "F.Cu" "B.Cu") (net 3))
 (segment (start 134.057 94.706328) (end 134.800672 95.45) (width 0.25) (layer "B.Cu") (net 3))
 (segment (start 134.800672 95.45) (end 139.25 95.45) (width 0.25) (layer "B.Cu") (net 3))
 (segment (start 139.25 95.45) (end 140.375 96.575) (width 0.25) (layer "B.Cu") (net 3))
 (segment (start 134.057 93.5) (end 134.057 94.706328) (width 0.25) (layer "B.Cu") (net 3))
 (segment (start 140.375 96.575) (end 140 96.95) (width 0.25) (layer "B.Cu") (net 3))
 (segment (start 140 96.95) (end 140 101.275) (width 0.25) (layer "B.Cu") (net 3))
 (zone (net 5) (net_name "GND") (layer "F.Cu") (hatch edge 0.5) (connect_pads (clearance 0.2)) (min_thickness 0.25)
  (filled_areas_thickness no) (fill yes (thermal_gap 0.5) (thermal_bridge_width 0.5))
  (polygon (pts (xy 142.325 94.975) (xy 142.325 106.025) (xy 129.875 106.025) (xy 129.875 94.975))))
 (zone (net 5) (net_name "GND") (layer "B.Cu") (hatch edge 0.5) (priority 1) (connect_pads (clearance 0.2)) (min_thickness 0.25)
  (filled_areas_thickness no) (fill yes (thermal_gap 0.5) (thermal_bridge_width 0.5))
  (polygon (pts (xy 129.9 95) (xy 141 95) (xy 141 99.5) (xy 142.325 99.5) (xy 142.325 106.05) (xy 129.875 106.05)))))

